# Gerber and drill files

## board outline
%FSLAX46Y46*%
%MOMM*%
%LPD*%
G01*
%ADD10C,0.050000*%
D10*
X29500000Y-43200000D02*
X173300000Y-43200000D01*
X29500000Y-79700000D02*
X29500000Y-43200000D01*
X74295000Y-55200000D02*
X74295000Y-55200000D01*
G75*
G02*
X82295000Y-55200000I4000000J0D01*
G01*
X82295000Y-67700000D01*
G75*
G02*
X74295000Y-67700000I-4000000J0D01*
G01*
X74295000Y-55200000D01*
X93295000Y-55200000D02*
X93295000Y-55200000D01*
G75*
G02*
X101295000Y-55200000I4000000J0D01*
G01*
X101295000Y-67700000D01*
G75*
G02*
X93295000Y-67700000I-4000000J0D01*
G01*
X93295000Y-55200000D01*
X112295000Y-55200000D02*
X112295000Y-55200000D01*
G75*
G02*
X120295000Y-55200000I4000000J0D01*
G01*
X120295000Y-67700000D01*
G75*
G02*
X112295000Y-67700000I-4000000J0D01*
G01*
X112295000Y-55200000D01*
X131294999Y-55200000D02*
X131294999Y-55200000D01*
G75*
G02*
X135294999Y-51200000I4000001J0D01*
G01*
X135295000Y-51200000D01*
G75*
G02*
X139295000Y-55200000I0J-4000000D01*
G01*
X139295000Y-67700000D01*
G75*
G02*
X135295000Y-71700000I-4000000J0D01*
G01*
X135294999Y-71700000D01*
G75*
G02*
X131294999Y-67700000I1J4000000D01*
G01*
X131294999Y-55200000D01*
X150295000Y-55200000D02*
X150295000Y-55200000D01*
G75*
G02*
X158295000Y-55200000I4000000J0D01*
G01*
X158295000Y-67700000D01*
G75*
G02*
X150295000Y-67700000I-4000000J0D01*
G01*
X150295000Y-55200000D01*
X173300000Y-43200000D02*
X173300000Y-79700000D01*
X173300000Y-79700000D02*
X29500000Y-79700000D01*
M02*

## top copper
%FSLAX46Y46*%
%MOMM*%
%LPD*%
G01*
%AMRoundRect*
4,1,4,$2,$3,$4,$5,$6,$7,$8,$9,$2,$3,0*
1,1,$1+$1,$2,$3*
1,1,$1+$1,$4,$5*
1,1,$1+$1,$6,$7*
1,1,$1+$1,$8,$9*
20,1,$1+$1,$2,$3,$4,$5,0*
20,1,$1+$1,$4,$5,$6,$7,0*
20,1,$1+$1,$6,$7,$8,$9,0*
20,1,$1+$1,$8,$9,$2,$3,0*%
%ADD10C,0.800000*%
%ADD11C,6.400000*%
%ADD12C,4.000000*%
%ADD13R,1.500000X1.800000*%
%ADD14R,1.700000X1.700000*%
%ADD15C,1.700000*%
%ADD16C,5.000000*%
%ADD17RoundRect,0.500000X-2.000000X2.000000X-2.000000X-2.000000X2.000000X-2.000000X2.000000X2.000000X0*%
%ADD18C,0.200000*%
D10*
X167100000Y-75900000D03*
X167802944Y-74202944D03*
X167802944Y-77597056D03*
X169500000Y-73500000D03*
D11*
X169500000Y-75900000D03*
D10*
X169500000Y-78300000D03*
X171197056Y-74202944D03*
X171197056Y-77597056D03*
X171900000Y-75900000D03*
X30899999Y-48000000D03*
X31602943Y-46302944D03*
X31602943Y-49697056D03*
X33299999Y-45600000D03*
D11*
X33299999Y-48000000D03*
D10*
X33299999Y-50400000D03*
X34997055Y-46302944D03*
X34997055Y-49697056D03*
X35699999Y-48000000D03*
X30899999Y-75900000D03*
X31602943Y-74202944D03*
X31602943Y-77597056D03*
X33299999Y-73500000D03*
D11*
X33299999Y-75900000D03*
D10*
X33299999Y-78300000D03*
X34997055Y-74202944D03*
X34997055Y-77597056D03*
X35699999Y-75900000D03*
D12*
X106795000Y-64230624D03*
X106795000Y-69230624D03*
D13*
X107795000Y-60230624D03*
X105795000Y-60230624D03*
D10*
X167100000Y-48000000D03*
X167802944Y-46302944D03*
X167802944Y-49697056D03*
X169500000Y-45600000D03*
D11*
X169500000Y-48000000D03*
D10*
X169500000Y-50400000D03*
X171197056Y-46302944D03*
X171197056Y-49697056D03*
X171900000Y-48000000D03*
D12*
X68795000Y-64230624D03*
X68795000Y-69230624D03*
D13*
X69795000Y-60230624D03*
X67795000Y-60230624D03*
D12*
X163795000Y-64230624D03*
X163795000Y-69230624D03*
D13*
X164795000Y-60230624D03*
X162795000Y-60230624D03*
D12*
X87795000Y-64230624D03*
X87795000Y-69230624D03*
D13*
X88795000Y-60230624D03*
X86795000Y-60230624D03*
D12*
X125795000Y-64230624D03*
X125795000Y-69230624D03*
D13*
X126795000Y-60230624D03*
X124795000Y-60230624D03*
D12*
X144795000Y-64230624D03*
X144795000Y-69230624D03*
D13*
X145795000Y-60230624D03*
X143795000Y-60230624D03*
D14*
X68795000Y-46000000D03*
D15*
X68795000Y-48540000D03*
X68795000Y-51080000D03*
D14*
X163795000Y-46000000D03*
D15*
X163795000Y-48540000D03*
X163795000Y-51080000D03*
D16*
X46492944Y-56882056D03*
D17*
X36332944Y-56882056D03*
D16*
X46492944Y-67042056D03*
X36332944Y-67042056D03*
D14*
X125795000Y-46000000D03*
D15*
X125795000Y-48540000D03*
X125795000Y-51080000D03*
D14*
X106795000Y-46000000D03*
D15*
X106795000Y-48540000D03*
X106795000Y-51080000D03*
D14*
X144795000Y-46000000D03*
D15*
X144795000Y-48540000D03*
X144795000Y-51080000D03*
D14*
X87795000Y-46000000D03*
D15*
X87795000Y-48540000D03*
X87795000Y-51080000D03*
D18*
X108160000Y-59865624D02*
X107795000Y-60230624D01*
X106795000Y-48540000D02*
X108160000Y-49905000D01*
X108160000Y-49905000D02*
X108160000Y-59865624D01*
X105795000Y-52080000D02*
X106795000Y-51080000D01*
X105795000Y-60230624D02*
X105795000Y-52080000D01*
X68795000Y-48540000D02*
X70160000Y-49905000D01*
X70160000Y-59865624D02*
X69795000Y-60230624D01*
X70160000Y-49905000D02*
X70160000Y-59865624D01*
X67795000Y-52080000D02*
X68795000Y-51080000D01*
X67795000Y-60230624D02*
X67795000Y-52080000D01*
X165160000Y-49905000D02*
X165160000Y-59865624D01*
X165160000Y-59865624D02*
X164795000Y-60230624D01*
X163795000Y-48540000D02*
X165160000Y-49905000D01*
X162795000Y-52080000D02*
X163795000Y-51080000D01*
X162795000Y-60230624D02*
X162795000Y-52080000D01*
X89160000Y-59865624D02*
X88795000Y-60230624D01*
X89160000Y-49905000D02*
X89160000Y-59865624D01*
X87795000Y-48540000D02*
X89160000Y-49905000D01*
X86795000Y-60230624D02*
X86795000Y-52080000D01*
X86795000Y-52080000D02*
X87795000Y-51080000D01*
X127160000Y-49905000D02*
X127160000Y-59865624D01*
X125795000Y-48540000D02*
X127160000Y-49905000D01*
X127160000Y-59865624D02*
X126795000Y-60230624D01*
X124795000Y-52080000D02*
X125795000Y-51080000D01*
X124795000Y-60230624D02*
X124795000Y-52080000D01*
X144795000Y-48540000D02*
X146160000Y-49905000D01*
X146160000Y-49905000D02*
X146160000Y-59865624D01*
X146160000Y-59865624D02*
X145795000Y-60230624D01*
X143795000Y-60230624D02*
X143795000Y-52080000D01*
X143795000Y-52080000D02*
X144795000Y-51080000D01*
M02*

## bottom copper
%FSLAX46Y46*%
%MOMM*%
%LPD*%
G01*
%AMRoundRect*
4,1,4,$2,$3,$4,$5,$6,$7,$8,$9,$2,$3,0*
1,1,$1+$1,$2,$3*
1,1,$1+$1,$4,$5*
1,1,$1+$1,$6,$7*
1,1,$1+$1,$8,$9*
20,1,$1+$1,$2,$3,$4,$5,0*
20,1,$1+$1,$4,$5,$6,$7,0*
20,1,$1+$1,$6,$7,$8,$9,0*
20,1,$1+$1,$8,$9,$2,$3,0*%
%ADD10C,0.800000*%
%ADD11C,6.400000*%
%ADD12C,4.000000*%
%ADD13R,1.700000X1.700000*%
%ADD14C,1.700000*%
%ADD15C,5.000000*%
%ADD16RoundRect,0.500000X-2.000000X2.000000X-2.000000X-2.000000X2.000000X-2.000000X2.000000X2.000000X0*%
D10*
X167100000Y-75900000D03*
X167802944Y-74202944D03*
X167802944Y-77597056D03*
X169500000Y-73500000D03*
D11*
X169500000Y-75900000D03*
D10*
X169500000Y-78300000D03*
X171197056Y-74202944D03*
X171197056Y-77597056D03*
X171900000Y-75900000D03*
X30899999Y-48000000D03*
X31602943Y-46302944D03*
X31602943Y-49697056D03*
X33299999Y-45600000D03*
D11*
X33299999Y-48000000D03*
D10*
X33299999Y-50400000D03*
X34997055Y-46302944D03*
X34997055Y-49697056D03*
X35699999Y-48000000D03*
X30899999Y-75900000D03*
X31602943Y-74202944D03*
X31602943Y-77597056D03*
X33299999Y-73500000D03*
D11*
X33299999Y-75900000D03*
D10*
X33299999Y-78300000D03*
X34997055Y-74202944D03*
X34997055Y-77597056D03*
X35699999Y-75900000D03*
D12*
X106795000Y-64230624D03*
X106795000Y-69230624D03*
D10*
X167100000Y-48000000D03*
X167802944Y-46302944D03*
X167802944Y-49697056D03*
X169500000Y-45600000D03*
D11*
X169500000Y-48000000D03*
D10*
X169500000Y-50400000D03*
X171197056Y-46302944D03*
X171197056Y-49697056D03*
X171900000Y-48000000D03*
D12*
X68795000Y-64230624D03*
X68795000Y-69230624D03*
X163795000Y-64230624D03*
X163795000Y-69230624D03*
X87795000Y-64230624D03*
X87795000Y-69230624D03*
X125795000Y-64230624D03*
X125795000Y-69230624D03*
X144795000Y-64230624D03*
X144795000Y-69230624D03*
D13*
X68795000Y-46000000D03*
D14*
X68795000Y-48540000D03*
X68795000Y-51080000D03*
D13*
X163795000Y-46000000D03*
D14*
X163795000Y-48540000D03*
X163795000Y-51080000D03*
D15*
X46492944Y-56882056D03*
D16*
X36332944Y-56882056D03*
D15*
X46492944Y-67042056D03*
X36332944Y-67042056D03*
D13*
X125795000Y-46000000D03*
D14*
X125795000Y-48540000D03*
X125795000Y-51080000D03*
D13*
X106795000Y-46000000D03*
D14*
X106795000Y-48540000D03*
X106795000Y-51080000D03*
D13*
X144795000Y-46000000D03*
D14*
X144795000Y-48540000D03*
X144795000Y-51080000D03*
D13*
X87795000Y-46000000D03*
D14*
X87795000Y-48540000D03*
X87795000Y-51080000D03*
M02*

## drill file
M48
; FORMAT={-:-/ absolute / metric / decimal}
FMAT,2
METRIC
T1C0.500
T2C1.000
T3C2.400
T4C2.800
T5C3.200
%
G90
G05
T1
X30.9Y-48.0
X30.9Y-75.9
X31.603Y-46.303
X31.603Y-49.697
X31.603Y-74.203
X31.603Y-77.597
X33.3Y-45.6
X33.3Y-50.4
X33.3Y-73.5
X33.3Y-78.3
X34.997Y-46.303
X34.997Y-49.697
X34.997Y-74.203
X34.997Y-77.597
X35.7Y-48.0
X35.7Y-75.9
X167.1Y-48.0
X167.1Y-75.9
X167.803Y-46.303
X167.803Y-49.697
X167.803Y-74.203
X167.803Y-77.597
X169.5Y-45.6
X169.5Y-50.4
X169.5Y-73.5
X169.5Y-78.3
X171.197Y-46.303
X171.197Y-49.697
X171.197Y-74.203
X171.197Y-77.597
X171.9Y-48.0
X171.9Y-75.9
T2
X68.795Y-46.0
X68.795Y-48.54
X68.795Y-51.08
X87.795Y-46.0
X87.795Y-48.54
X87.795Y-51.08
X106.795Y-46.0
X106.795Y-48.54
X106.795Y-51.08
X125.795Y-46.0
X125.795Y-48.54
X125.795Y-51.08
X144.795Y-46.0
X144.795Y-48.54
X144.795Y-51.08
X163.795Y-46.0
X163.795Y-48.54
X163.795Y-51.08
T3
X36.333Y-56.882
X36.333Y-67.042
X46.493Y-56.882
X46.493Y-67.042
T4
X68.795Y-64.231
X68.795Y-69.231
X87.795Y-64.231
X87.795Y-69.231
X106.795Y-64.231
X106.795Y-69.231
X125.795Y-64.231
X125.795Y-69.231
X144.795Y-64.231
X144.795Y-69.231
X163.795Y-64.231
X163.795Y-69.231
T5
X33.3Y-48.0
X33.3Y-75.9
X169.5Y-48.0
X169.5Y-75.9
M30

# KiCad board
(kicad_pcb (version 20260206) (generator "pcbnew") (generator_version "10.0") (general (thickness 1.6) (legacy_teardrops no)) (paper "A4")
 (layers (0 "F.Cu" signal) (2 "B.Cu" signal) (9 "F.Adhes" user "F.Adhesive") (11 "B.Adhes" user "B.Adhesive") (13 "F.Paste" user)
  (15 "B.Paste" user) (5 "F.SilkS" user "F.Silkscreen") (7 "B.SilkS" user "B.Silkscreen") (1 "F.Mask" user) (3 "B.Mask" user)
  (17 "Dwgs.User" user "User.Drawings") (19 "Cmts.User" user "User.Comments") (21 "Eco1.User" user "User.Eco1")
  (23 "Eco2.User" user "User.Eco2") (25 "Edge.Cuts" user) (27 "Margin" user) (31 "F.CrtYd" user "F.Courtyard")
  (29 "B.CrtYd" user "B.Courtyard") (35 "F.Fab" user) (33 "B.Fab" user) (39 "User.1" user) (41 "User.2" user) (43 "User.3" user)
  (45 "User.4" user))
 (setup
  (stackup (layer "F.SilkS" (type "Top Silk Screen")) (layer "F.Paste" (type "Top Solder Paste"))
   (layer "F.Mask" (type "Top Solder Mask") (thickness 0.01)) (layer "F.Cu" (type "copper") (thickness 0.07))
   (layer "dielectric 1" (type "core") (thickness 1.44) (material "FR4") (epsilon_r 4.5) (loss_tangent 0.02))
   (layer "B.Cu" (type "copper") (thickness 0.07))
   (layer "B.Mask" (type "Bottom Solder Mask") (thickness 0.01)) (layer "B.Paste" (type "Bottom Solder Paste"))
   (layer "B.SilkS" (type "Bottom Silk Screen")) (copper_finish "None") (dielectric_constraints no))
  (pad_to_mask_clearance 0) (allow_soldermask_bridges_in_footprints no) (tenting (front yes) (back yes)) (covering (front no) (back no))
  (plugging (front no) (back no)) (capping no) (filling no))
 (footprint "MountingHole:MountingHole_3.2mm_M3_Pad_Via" (layer "F.Cu") (at 169.5 75.9)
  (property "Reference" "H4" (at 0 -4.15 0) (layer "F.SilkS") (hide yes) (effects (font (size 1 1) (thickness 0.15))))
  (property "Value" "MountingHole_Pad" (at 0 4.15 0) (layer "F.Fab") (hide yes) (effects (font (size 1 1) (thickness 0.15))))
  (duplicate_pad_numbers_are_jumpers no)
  (pad "1" thru_hole circle (at -2.4 0) (size 0.8 0.8) (drill 0.5) (layers "*.Cu" "*.Mask") (remove_unused_layers no) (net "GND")
   (zone_connect 2))
  (pad "1" thru_hole circle (at -1.697056 -1.697056) (size 0.8 0.8) (drill 0.5) (layers "*.Cu" "*.Mask") (remove_unused_layers no)
   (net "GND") (zone_connect 2))
  (pad "1" thru_hole circle (at -1.697056 1.697056) (size 0.8 0.8) (drill 0.5) (layers "*.Cu" "*.Mask") (remove_unused_layers no)
   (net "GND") (zone_connect 2))
  (pad "1" thru_hole circle (at 0 -2.4) (size 0.8 0.8) (drill 0.5) (layers "*.Cu" "*.Mask") (remove_unused_layers no) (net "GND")
   (zone_connect 2))
  (pad "1" thru_hole circle (at 0 0) (size 6.4 6.4) (drill 3.2) (layers "*.Cu" "*.Mask") (remove_unused_layers no) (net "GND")
   (zone_connect 2))
  (pad "1" thru_hole circle (at 0 2.4) (size 0.8 0.8) (drill 0.5) (layers "*.Cu" "*.Mask") (remove_unused_layers no) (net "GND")
   (zone_connect 2))
  (pad "1" thru_hole circle (at 1.697056 -1.697056) (size 0.8 0.8) (drill 0.5) (layers "*.Cu" "*.Mask") (remove_unused_layers no)
   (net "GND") (zone_connect 2))
  (pad "1" thru_hole circle (at 1.697056 1.697056) (size 0.8 0.8) (drill 0.5) (layers "*.Cu" "*.Mask") (remove_unused_layers no) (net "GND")
   (zone_connect 2))
  (pad "1" thru_hole circle (at 2.4 0) (size 0.8 0.8) (drill 0.5) (layers "*.Cu" "*.Mask") (remove_unused_layers no) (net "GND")
   (zone_connect 2)))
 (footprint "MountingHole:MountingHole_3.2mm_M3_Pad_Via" (layer "F.Cu") (at 33.299999 48)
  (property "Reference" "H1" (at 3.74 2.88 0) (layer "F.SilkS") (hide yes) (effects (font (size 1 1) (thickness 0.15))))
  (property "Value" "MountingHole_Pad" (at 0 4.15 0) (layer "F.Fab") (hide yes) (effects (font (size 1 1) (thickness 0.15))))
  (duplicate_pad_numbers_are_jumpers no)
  (pad "1" thru_hole circle (at -2.4 0) (size 0.8 0.8) (drill 0.5) (layers "*.Cu" "*.Mask") (remove_unused_layers no) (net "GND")
   (zone_connect 2))
  (pad "1" thru_hole circle (at -1.697056 -1.697056) (size 0.8 0.8) (drill 0.5) (layers "*.Cu" "*.Mask") (remove_unused_layers no)
   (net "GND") (zone_connect 2))
  (pad "1" thru_hole circle (at -1.697056 1.697056) (size 0.8 0.8) (drill 0.5) (layers "*.Cu" "*.Mask") (remove_unused_layers no)
   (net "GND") (zone_connect 2))
  (pad "1" thru_hole circle (at 0 -2.4) (size 0.8 0.8) (drill 0.5) (layers "*.Cu" "*.Mask") (remove_unused_layers no) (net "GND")
   (zone_connect 2))
  (pad "1" thru_hole circle (at 0 0) (size 6.4 6.4) (drill 3.2) (layers "*.Cu" "*.Mask") (remove_unused_layers no) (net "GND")
   (zone_connect 2))
  (pad "1" thru_hole circle (at 0 2.4) (size 0.8 0.8) (drill 0.5) (layers "*.Cu" "*.Mask") (remove_unused_layers no) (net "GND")
   (zone_connect 2))
  (pad "1" thru_hole circle (at 1.697056 -1.697056) (size 0.8 0.8) (drill 0.5) (layers "*.Cu" "*.Mask") (remove_unused_layers no)
   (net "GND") (zone_connect 2))
  (pad "1" thru_hole circle (at 1.697056 1.697056) (size 0.8 0.8) (drill 0.5) (layers "*.Cu" "*.Mask") (remove_unused_layers no) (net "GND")
   (zone_connect 2))
  (pad "1" thru_hole circle (at 2.4 0) (size 0.8 0.8) (drill 0.5) (layers "*.Cu" "*.Mask") (remove_unused_layers no) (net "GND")
   (zone_connect 2)))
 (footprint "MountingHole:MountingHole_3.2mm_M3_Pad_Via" (layer "F.Cu") (at 33.299999 75.9)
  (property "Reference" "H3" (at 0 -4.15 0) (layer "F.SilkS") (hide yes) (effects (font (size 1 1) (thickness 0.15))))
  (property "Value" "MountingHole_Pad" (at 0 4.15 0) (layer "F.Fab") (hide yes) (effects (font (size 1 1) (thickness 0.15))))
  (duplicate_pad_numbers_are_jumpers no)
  (pad "1" thru_hole circle (at -2.4 0) (size 0.8 0.8) (drill 0.5) (layers "*.Cu" "*.Mask") (remove_unused_layers no) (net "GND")
   (zone_connect 2))
  (pad "1" thru_hole circle (at -1.697056 -1.697056) (size 0.8 0.8) (drill 0.5) (layers "*.Cu" "*.Mask") (remove_unused_layers no)
   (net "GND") (zone_connect 2))
  (pad "1" thru_hole circle (at -1.697056 1.697056) (size 0.8 0.8) (drill 0.5) (layers "*.Cu" "*.Mask") (remove_unused_layers no)
   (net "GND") (zone_connect 2))
  (pad "1" thru_hole circle (at 0 -2.4) (size 0.8 0.8) (drill 0.5) (layers "*.Cu" "*.Mask") (remove_unused_layers no) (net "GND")
   (zone_connect 2))
  (pad "1" thru_hole circle (at 0 0) (size 6.4 6.4) (drill 3.2) (layers "*.Cu" "*.Mask") (remove_unused_layers no) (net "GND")
   (zone_connect 2))
  (pad "1" thru_hole circle (at 0 2.4) (size 0.8 0.8) (drill 0.5) (layers "*.Cu" "*.Mask") (remove_unused_layers no) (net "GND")
   (zone_connect 2))
  (pad "1" thru_hole circle (at 1.697056 -1.697056) (size 0.8 0.8) (drill 0.5) (layers "*.Cu" "*.Mask") (remove_unused_layers no)
   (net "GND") (zone_connect 2))
  (pad "1" thru_hole circle (at 1.697056 1.697056) (size 0.8 0.8) (drill 0.5) (layers "*.Cu" "*.Mask") (remove_unused_layers no) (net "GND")
   (zone_connect 2))
  (pad "1" thru_hole circle (at 2.4 0) (size 0.8 0.8) (drill 0.5) (layers "*.Cu" "*.Mask") (remove_unused_layers no) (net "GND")
   (zone_connect 2)))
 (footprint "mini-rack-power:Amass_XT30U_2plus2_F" (layer "F.Cu") (at 106.795 64.91 -90)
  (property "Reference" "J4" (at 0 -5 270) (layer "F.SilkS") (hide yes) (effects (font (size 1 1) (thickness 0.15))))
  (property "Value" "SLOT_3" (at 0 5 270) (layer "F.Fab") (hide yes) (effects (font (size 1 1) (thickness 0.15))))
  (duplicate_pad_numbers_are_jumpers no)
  (pad "1" thru_hole circle (at -0.679376 0 270) (size 4 4) (drill 2.8) (layers "*.Cu" "*.Mask") (remove_unused_layers no) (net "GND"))
  (pad "2" thru_hole circle (at 4.320624 0 270) (size 4 4) (drill 2.8) (layers "*.Cu" "*.Mask") (remove_unused_layers no) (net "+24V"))
  (pad "3" smd rect (at -4.679376 -1 270) (size 1.8 1.5) (layers "F.Cu" "F.Mask" "F.Paste") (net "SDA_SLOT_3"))
  (pad "4" smd rect (at -4.679376 1 270) (size 1.8 1.5) (layers "F.Cu" "F.Mask" "F.Paste") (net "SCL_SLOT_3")))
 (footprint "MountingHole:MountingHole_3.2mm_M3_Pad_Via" (layer "F.Cu") (at 169.5 48)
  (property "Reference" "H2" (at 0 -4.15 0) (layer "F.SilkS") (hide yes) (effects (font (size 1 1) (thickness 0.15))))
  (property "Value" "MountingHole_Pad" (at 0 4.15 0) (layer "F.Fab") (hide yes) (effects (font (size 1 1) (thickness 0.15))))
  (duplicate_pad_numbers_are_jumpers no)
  (pad "1" thru_hole circle (at -2.4 0) (size 0.8 0.8) (drill 0.5) (layers "*.Cu" "*.Mask") (remove_unused_layers no) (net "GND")
   (zone_connect 2))
  (pad "1" thru_hole circle (at -1.697056 -1.697056) (size 0.8 0.8) (drill 0.5) (layers "*.Cu" "*.Mask") (remove_unused_layers no)
   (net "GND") (zone_connect 2))
  (pad "1" thru_hole circle (at -1.697056 1.697056) (size 0.8 0.8) (drill 0.5) (layers "*.Cu" "*.Mask") (remove_unused_layers no)
   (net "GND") (zone_connect 2))
  (pad "1" thru_hole circle (at 0 -2.4) (size 0.8 0.8) (drill 0.5) (layers "*.Cu" "*.Mask") (remove_unused_layers no) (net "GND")
   (zone_connect 2))
  (pad "1" thru_hole circle (at 0 0) (size 6.4 6.4) (drill 3.2) (layers "*.Cu" "*.Mask") (remove_unused_layers no) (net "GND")
   (zone_connect 2))
  (pad "1" thru_hole circle (at 0 2.4) (size 0.8 0.8) (drill 0.5) (layers "*.Cu" "*.Mask") (remove_unused_layers no) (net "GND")
   (zone_connect 2))
  (pad "1" thru_hole circle (at 1.697056 -1.697056) (size 0.8 0.8) (drill 0.5) (layers "*.Cu" "*.Mask") (remove_unused_layers no)
   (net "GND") (zone_connect 2))
  (pad "1" thru_hole circle (at 1.697056 1.697056) (size 0.8 0.8) (drill 0.5) (layers "*.Cu" "*.Mask") (remove_unused_layers no) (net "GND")
   (zone_connect 2))
  (pad "1" thru_hole circle (at 2.4 0) (size 0.8 0.8) (drill 0.5) (layers "*.Cu" "*.Mask") (remove_unused_layers no) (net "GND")
   (zone_connect 2)))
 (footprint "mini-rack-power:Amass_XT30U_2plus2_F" (layer "F.Cu") (at 68.795 64.91 -90)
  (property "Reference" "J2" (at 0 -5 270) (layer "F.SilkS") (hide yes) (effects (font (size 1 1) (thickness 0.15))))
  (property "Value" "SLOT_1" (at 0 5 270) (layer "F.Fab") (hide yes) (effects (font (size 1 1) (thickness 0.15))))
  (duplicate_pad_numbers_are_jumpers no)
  (pad "1" thru_hole circle (at -0.679376 0 270) (size 4 4) (drill 2.8) (layers "*.Cu" "*.Mask") (remove_unused_layers no) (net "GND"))
  (pad "2" thru_hole circle (at 4.320624 0 270) (size 4 4) (drill 2.8) (layers "*.Cu" "*.Mask") (remove_unused_layers no) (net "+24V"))
  (pad "3" smd rect (at -4.679376 -1 270) (size 1.8 1.5) (layers "F.Cu" "F.Mask" "F.Paste") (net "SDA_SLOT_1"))
  (pad "4" smd rect (at -4.679376 1 270) (size 1.8 1.5) (layers "F.Cu" "F.Mask" "F.Paste") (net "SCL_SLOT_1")))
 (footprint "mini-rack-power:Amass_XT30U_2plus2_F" (layer "F.Cu") (at 163.795 64.91 -90)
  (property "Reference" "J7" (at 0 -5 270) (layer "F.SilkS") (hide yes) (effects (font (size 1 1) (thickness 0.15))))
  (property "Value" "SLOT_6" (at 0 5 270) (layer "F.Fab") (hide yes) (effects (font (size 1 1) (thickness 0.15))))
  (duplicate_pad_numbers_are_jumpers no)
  (pad "1" thru_hole circle (at -0.679376 0 270) (size 4 4) (drill 2.8) (layers "*.Cu" "*.Mask") (remove_unused_layers no) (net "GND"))
  (pad "2" thru_hole circle (at 4.320624 0 270) (size 4 4) (drill 2.8) (layers "*.Cu" "*.Mask") (remove_unused_layers no) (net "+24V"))
  (pad "3" smd rect (at -4.679376 -1 270) (size 1.8 1.5) (layers "F.Cu" "F.Mask" "F.Paste") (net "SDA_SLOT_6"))
  (pad "4" smd rect (at -4.679376 1 270) (size 1.8 1.5) (layers "F.Cu" "F.Mask" "F.Paste") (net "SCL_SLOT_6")))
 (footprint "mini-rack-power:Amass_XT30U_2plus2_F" (layer "F.Cu") (at 87.795 64.91 -90)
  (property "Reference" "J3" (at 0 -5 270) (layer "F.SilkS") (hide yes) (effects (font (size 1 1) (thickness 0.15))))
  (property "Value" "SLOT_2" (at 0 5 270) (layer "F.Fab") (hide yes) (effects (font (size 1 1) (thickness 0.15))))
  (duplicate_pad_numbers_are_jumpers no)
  (pad "1" thru_hole circle (at -0.679376 0 270) (size 4 4) (drill 2.8) (layers "*.Cu" "*.Mask") (remove_unused_layers no) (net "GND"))
  (pad "2" thru_hole circle (at 4.320624 0 270) (size 4 4) (drill 2.8) (layers "*.Cu" "*.Mask") (remove_unused_layers no) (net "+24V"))
  (pad "3" smd rect (at -4.679376 -1 270) (size 1.8 1.5) (layers "F.Cu" "F.Mask" "F.Paste") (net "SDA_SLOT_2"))
  (pad "4" smd rect (at -4.679376 1 270) (size 1.8 1.5) (layers "F.Cu" "F.Mask" "F.Paste") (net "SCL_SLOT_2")))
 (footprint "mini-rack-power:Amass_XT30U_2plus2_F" (layer "F.Cu") (at 125.795 64.91 -90)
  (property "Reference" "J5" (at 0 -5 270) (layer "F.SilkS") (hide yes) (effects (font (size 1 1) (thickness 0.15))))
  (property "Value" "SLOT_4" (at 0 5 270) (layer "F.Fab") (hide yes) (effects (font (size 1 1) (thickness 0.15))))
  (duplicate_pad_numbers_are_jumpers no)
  (pad "1" thru_hole circle (at -0.679376 0 270) (size 4 4) (drill 2.8) (layers "*.Cu" "*.Mask") (remove_unused_layers no) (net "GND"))
  (pad "2" thru_hole circle (at 4.320624 0 270) (size 4 4) (drill 2.8) (layers "*.Cu" "*.Mask") (remove_unused_layers no) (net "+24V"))
  (pad "3" smd rect (at -4.679376 -1 270) (size 1.8 1.5) (layers "F.Cu" "F.Mask" "F.Paste") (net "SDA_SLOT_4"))
  (pad "4" smd rect (at -4.679376 1 270) (size 1.8 1.5) (layers "F.Cu" "F.Mask" "F.Paste") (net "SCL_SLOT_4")))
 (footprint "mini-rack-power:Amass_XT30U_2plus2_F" (layer "F.Cu") (at 144.795 64.91 -90)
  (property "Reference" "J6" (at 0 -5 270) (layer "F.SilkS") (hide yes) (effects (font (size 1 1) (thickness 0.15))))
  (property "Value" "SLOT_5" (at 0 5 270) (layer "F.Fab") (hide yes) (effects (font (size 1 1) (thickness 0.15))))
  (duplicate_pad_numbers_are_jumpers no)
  (pad "1" thru_hole circle (at -0.679376 0 270) (size 4 4) (drill 2.8) (layers "*.Cu" "*.Mask") (remove_unused_layers no) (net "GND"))
  (pad "2" thru_hole circle (at 4.320624 0 270) (size 4 4) (drill 2.8) (layers "*.Cu" "*.Mask") (remove_unused_layers no) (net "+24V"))
  (pad "3" smd rect (at -4.679376 -1 270) (size 1.8 1.5) (layers "F.Cu" "F.Mask" "F.Paste") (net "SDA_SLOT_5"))
  (pad "4" smd rect (at -4.679376 1 270) (size 1.8 1.5) (layers "F.Cu" "F.Mask" "F.Paste") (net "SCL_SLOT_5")))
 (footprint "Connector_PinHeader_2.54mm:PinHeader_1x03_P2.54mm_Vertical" (layer "B.Cu") (at 68.795 46 180)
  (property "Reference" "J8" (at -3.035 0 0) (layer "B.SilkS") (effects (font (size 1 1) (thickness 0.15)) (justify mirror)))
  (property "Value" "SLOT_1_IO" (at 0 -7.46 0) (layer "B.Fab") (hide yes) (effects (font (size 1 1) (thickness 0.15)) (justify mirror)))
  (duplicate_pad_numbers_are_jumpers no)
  (pad "1" thru_hole rect (at 0 0 180) (size 1.7 1.7) (drill 1) (layers "*.Cu" "*.Mask") (remove_unused_layers no) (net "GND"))
  (pad "2" thru_hole circle (at 0 -2.54 180) (size 1.7 1.7) (drill 1) (layers "*.Cu" "*.Mask") (remove_unused_layers no) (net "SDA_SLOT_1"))
  (pad "3" thru_hole circle (at 0 -5.08 180) (size 1.7 1.7) (drill 1) (layers "*.Cu" "*.Mask") (remove_unused_layers no) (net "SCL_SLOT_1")))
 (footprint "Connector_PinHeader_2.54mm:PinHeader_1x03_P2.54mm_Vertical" (layer "B.Cu") (at 163.795 46 180)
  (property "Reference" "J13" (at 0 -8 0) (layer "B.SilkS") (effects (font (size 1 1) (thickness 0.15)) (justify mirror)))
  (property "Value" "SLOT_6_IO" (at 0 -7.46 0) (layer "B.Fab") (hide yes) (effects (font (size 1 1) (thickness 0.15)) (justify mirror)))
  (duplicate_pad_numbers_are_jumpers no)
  (pad "1" thru_hole rect (at 0 0 180) (size 1.7 1.7) (drill 1) (layers "*.Cu" "*.Mask") (remove_unused_layers no) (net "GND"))
  (pad "2" thru_hole circle (at 0 -2.54 180) (size 1.7 1.7) (drill 1) (layers "*.Cu" "*.Mask") (remove_unused_layers no) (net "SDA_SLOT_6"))
  (pad "3" thru_hole circle (at 0 -5.08 180) (size 1.7 1.7) (drill 1) (layers "*.Cu" "*.Mask") (remove_unused_layers no) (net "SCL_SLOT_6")))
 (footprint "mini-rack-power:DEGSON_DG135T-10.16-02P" (layer "B.Cu") (at 36.332944 56.882056 -90)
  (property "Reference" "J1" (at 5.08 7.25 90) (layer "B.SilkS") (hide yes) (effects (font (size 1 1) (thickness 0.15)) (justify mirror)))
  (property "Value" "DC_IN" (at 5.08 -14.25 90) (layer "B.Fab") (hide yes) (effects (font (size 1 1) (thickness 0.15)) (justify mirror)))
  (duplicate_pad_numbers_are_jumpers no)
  (pad "1" thru_hole circle (at 0 -10.16 270) (size 5 5) (drill 2.4) (layers "*.Cu" "*.Mask") (remove_unused_layers no) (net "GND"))
  (pad "1" thru_hole roundrect (at 0 0 270) (size 5 5) (drill 2.4) (layers "*.Cu" "*.Mask") (remove_unused_layers no) (roundrect_rratio 0.1)
   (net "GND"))
  (pad "2" thru_hole circle (at 10.16 -10.16 270) (size 5 5) (drill 2.4) (layers "*.Cu" "*.Mask") (remove_unused_layers no) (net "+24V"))
  (pad "2" thru_hole circle (at 10.16 0 270) (size 5 5) (drill 2.4) (layers "*.Cu" "*.Mask") (remove_unused_layers no) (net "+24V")))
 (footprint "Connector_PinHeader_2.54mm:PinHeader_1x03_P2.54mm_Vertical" (layer "B.Cu") (at 125.795 46 180)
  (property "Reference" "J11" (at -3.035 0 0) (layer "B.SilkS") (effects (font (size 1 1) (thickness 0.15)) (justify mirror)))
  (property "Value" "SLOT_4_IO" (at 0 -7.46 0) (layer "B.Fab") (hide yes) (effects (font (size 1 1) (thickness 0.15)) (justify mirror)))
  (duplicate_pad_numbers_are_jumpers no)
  (pad "1" thru_hole rect (at 0 0 180) (size 1.7 1.7) (drill 1) (layers "*.Cu" "*.Mask") (remove_unused_layers no) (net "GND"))
  (pad "2" thru_hole circle (at 0 -2.54 180) (size 1.7 1.7) (drill 1) (layers "*.Cu" "*.Mask") (remove_unused_layers no) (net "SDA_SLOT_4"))
  (pad "3" thru_hole circle (at 0 -5.08 180) (size 1.7 1.7) (drill 1) (layers "*.Cu" "*.Mask") (remove_unused_layers no) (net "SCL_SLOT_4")))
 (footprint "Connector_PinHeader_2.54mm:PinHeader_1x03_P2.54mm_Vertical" (layer "B.Cu") (at 106.795 46 180)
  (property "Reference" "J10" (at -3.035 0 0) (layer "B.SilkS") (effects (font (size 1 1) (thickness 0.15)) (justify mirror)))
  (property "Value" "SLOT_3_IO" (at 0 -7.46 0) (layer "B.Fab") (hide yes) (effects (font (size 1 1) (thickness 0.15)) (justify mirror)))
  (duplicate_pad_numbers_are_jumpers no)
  (pad "1" thru_hole rect (at 0 0 180) (size 1.7 1.7) (drill 1) (layers "*.Cu" "*.Mask") (remove_unused_layers no) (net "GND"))
  (pad "2" thru_hole circle (at 0 -2.54 180) (size 1.7 1.7) (drill 1) (layers "*.Cu" "*.Mask") (remove_unused_layers no) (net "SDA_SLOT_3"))
  (pad "3" thru_hole circle (at 0 -5.08 180) (size 1.7 1.7) (drill 1) (layers "*.Cu" "*.Mask") (remove_unused_layers no) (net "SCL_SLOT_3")))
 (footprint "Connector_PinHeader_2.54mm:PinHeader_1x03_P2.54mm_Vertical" (layer "B.Cu") (at 144.795 46 180)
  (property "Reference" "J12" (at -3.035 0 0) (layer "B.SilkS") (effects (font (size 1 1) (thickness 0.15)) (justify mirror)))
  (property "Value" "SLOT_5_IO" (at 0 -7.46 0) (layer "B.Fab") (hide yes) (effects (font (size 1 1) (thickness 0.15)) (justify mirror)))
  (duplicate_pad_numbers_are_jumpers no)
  (pad "1" thru_hole rect (at 0 0 180) (size 1.7 1.7) (drill 1) (layers "*.Cu" "*.Mask") (remove_unused_layers no) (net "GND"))
  (pad "2" thru_hole circle (at 0 -2.54 180) (size 1.7 1.7) (drill 1) (layers "*.Cu" "*.Mask") (remove_unused_layers no) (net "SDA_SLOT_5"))
  (pad "3" thru_hole circle (at 0 -5.08 180) (size 1.7 1.7) (drill 1) (layers "*.Cu" "*.Mask") (remove_unused_layers no) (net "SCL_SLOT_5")))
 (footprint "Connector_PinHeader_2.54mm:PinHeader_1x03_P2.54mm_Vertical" (layer "B.Cu") (at 87.795 46 180)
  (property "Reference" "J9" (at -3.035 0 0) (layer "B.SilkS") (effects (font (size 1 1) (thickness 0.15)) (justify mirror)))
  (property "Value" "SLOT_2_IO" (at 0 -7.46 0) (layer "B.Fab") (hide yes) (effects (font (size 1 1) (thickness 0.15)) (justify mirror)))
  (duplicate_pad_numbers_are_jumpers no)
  (pad "1" thru_hole rect (at 0 0 180) (size 1.7 1.7) (drill 1) (layers "*.Cu" "*.Mask") (remove_unused_layers no) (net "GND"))
  (pad "2" thru_hole circle (at 0 -2.54 180) (size 1.7 1.7) (drill 1) (layers "*.Cu" "*.Mask") (remove_unused_layers no) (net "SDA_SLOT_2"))
  (pad "3" thru_hole circle (at 0 -5.08 180) (size 1.7 1.7) (drill 1) (layers "*.Cu" "*.Mask") (remove_unused_layers no) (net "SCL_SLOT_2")))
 (gr_line (start 29.5 43.2) (end 173.3 43.2) (stroke (width 0.05) (type default)) (layer "Edge.Cuts"))
 (gr_line (start 29.5 79.7) (end 29.5 43.2) (stroke (width 0.05) (type default)) (layer "Edge.Cuts"))
 (gr_rect (start 74.295 51.2) (end 82.295 71.7) (radius 4) (stroke (width 0.05) (type default)) (fill no) (layer "Edge.Cuts"))
 (gr_rect (start 93.295 51.2) (end 101.295 71.7) (radius 4) (stroke (width 0.05) (type default)) (fill no) (layer "Edge.Cuts"))
 (gr_rect (start 112.295 51.2) (end 120.295 71.7) (radius 4) (stroke (width 0.05) (type default)) (fill no) (layer "Edge.Cuts"))
 (gr_rect (start 131.294999 51.2) (end 139.295 71.7) (radius 4) (stroke (width 0.05) (type default)) (fill no) (layer "Edge.Cuts"))
 (gr_rect (start 150.295 51.2) (end 158.295 71.7) (radius 4) (stroke (width 0.05) (type default)) (fill no) (layer "Edge.Cuts"))
 (gr_line (start 173.3 43.2) (end 173.3 79.7) (stroke (width 0.05) (type default)) (layer "Edge.Cuts"))
 (gr_line (start 173.3 79.7) (end 29.5 79.7) (stroke (width 0.05) (type default)) (layer "Edge.Cuts"))
 (segment (start 108.16 59.865624) (end 107.795 60.230624) (width 0.2) (layer "F.Cu") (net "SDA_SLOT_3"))
 (segment (start 106.795 48.54) (end 108.16 49.905) (width 0.2) (layer "F.Cu") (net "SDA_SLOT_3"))
 (segment (start 108.16 49.905) (end 108.16 59.865624) (width 0.2) (layer "F.Cu") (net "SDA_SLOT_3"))
 (segment (start 105.795 52.08) (end 106.795 51.08) (width 0.2) (layer "F.Cu") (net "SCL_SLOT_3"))
 (segment (start 105.795 60.230624) (end 105.795 52.08) (width 0.2) (layer "F.Cu") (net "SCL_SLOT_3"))
 (segment (start 68.795 48.54) (end 70.16 49.905) (width 0.2) (layer "F.Cu") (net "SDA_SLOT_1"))
 (segment (start 70.16 59.865624) (end 69.795 60.230624) (width 0.2) (layer "F.Cu") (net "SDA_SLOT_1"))
 (segment (start 70.16 49.905) (end 70.16 59.865624) (width 0.2) (layer "F.Cu") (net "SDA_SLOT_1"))
 (segment (start 67.795 52.08) (end 68.795 51.08) (width 0.2) (layer "F.Cu") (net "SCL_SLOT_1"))
 (segment (start 67.795 60.230624) (end 67.795 52.08) (width 0.2) (layer "F.Cu") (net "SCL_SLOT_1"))
 (segment (start 165.16 49.905) (end 165.16 59.865624) (width 0.2) (layer "F.Cu") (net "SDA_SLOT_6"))
 (segment (start 165.16 59.865624) (end 164.795 60.230624) (width 0.2) (layer "F.Cu") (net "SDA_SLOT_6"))
 (segment (start 163.795 48.54) (end 165.16 49.905) (width 0.2) (layer "F.Cu") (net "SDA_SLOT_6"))
 (segment (start 162.795 52.08) (end 163.795 51.08) (width 0.2) (layer "F.Cu") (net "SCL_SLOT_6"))
 (segment (start 162.795 60.230624) (end 162.795 52.08) (width 0.2) (layer "F.Cu") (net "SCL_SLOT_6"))
 (segment (start 89.16 59.865624) (end 88.795 60.230624) (width 0.2) (layer "F.Cu") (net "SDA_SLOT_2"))
 (segment (start 89.16 49.905) (end 89.16 59.865624) (width 0.2) (layer "F.Cu") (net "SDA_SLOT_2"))
 (segment (start 87.795 48.54) (end 89.16 49.905) (width 0.2) (layer "F.Cu") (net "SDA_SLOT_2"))
 (segment (start 86.795 60.230624) (end 86.795 52.08) (width 0.2) (layer "F.Cu") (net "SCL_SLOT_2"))
 (segment (start 86.795 52.08) (end 87.795 51.08) (width 0.2) (layer "F.Cu") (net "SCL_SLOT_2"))
 (segment (start 127.16 49.905) (end 127.16 59.865624) (width 0.2) (layer "F.Cu") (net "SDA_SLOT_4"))
 (segment (start 125.795 48.54) (end 127.16 49.905) (width 0.2) (layer "F.Cu") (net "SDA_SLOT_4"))
 (segment (start 127.16 59.865624) (end 126.795 60.230624) (width 0.2) (layer "F.Cu") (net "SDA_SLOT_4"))
 (segment (start 124.795 52.08) (end 125.795 51.08) (width 0.2) (layer "F.Cu") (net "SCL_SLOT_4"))
 (segment (start 124.795 60.230624) (end 124.795 52.08) (width 0.2) (layer "F.Cu") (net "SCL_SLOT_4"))
 (segment (start 144.795 48.54) (end 146.16 49.905) (width 0.2) (layer "F.Cu") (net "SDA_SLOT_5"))
 (segment (start 146.16 49.905) (end 146.16 59.865624) (width 0.2) (layer "F.Cu") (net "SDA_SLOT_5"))
 (segment (start 146.16 59.865624) (end 145.795 60.230624) (width 0.2) (layer "F.Cu") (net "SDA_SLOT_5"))
 (segment (start 143.795 60.230624) (end 143.795 52.08) (width 0.2) (layer "F.Cu") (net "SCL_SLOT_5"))
 (segment (start 143.795 52.08) (end 144.795 51.08) (width 0.2) (layer "F.Cu") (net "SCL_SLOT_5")))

